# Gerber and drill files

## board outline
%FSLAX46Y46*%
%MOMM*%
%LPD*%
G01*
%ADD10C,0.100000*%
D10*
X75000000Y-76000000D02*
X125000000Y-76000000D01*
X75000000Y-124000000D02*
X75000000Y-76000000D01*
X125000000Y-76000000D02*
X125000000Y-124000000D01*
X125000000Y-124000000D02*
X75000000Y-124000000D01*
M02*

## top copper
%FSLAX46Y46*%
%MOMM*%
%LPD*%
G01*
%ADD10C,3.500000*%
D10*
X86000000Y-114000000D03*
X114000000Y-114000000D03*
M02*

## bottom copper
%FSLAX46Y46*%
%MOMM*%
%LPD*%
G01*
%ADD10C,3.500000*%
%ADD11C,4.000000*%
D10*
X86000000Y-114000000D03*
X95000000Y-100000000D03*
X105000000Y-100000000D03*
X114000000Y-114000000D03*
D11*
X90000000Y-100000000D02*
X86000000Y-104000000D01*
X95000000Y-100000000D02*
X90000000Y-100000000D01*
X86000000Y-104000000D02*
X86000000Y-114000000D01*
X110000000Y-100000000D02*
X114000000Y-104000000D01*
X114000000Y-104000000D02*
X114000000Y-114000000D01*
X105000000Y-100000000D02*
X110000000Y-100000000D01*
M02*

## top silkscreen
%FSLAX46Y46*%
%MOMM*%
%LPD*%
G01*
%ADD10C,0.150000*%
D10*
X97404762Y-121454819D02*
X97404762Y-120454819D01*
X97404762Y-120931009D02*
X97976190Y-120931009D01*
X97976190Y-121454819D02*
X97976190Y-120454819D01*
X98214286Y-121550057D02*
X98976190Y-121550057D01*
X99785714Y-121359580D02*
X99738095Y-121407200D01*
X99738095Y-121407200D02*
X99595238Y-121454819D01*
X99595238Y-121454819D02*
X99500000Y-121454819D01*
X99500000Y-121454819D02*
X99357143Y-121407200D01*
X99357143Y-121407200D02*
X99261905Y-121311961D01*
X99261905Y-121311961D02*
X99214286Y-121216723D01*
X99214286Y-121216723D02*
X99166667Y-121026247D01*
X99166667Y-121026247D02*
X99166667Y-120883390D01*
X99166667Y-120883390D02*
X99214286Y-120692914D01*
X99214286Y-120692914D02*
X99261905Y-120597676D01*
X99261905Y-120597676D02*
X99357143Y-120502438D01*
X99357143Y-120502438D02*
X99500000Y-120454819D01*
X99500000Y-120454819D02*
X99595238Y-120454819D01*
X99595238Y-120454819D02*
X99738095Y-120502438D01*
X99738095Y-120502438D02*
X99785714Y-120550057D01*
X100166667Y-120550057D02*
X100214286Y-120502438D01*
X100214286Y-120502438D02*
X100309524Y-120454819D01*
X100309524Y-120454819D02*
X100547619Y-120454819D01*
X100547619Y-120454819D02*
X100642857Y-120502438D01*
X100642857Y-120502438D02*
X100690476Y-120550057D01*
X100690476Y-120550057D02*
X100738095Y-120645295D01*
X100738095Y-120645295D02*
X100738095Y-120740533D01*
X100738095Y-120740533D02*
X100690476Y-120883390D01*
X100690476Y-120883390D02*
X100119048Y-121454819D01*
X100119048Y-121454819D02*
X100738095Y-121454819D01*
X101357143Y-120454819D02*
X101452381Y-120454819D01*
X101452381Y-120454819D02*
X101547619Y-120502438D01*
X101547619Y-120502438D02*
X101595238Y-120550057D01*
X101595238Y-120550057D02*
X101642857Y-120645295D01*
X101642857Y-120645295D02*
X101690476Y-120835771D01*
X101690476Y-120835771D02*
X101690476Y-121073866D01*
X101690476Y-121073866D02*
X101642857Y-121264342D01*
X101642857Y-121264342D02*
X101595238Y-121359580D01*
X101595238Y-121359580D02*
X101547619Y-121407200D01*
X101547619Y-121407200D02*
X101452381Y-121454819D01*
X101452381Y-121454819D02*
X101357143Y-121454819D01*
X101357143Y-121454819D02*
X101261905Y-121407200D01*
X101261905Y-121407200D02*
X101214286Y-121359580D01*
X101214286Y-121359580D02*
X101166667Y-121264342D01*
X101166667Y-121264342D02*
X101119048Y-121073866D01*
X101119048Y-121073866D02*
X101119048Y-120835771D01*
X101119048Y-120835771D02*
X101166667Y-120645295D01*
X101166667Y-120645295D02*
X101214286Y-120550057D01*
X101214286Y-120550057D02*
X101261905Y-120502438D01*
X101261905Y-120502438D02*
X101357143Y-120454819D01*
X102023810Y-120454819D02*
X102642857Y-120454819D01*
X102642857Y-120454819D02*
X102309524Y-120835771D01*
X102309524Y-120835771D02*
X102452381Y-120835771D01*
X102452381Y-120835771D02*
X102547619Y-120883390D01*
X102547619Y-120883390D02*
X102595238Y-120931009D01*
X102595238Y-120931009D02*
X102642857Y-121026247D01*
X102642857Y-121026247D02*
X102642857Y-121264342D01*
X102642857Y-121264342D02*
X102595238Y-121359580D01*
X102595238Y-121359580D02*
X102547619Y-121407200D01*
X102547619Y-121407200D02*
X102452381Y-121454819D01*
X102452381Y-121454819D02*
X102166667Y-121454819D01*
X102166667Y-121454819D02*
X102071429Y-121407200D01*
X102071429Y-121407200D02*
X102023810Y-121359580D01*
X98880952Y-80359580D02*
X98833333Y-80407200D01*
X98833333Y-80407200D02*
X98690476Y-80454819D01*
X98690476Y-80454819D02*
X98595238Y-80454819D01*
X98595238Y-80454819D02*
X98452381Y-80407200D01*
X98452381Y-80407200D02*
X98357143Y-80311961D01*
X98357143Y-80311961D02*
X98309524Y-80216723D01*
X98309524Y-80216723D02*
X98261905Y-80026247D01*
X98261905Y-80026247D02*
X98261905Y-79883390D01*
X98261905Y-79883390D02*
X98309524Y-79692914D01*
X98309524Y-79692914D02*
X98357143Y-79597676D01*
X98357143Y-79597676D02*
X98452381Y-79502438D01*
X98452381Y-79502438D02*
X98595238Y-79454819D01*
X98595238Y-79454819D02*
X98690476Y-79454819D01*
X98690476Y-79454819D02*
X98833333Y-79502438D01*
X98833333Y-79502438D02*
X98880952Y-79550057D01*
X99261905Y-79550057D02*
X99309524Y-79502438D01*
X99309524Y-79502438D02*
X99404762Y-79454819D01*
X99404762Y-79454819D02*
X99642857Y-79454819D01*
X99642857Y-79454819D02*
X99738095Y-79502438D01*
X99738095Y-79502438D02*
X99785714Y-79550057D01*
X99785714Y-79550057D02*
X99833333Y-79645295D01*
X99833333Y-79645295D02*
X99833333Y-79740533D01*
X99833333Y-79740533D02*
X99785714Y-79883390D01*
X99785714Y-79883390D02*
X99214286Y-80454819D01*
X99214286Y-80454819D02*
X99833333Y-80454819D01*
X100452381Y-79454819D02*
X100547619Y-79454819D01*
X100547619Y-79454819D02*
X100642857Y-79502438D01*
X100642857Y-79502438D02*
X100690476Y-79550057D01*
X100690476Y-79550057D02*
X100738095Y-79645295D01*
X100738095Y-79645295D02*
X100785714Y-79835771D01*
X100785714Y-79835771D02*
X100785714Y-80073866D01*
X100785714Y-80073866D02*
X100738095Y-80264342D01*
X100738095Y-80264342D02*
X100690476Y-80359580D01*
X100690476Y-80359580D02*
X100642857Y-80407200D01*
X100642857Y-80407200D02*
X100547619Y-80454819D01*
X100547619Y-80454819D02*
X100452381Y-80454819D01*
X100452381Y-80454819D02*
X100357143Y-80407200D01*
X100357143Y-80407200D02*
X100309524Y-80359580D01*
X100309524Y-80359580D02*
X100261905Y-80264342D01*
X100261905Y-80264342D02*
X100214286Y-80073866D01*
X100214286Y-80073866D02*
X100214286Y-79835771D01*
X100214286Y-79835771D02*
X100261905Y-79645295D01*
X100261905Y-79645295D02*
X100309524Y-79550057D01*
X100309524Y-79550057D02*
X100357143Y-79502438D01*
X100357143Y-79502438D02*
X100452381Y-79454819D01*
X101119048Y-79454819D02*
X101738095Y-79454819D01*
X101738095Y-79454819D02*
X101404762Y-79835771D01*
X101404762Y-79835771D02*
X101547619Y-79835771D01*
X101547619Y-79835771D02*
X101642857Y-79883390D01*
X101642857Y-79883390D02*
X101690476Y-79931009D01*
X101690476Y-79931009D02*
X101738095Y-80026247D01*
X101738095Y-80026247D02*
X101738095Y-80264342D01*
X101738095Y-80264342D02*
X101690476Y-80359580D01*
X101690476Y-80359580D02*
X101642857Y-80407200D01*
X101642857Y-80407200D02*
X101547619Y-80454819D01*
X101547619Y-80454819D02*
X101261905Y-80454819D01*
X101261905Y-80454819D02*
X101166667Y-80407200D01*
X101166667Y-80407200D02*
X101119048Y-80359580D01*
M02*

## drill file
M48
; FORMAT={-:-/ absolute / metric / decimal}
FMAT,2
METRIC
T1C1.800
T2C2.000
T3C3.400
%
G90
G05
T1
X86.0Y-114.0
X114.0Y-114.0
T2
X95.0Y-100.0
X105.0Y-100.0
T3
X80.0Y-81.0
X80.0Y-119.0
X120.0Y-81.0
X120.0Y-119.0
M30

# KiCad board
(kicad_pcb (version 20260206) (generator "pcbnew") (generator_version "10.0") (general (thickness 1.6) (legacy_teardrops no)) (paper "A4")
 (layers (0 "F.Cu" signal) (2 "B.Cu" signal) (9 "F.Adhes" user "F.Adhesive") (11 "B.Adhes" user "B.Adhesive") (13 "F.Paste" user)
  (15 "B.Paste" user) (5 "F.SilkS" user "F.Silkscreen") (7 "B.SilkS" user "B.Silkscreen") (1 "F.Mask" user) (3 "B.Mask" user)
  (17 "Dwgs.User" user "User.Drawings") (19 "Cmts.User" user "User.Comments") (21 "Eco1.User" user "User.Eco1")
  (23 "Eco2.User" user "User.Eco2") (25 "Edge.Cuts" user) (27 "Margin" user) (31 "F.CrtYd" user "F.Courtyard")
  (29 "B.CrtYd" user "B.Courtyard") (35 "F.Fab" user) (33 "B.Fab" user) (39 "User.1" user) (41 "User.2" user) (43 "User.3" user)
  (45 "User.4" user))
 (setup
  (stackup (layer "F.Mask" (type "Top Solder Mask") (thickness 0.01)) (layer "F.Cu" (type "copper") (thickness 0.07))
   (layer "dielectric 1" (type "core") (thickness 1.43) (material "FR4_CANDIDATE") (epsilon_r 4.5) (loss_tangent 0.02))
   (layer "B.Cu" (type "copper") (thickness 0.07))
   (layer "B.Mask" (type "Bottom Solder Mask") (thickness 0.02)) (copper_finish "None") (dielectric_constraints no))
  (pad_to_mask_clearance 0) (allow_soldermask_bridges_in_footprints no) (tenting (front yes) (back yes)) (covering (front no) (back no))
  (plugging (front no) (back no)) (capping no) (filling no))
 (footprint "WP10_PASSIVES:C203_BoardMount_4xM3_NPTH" (layer "F.Cu") (at 100 100)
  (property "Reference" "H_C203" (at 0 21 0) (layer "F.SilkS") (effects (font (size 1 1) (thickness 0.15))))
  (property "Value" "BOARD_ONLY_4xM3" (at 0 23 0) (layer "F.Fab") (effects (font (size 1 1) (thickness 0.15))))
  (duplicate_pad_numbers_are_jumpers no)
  (pad "" np_thru_hole circle (at -20 -19) (size 3.4 3.4) (drill 3.4) (layers "*.Cu" "*.Mask"))
  (pad "" np_thru_hole circle (at -20 19) (size 3.4 3.4) (drill 3.4) (layers "*.Cu" "*.Mask"))
  (pad "" np_thru_hole circle (at 20 -19) (size 3.4 3.4) (drill 3.4) (layers "*.Cu" "*.Mask"))
  (pad "" np_thru_hole circle (at 20 19) (size 3.4 3.4) (drill 3.4) (layers "*.Cu" "*.Mask")))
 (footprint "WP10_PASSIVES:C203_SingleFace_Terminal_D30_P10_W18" (layer "F.Cu") (at 100 100)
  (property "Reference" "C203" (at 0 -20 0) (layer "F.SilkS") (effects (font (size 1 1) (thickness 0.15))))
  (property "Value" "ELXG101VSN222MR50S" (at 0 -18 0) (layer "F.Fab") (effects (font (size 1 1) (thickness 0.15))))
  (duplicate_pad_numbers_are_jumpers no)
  (pad "1" thru_hole circle (at -14 14) (size 3.5 3.5) (drill 1.8) (layers "*.Cu" "*.Mask") (remove_unused_layers no)
   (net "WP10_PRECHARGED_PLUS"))
  (pad "1" thru_hole circle (at -5 0) (size 3.5 3.5) (drill 2) (layers "*.Cu" "*.Mask") (remove_unused_layers yes) (keep_end_layers no)
   (zone_layer_connections) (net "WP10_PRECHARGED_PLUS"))
  (pad "2" thru_hole circle (at 5 0) (size 3.5 3.5) (drill 2) (layers "*.Cu" "*.Mask") (remove_unused_layers yes) (keep_end_layers no)
   (zone_layer_connections) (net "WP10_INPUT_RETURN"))
  (pad "2" thru_hole circle (at 14 14) (size 3.5 3.5) (drill 1.8) (layers "*.Cu" "*.Mask") (remove_unused_layers no)
   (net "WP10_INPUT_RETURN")))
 (gr_line (start 75 76) (end 125 76) (stroke (width 0.1) (type default)) (layer "Edge.Cuts"))
 (gr_line (start 75 124) (end 75 76) (stroke (width 0.1) (type default)) (layer "Edge.Cuts"))
 (gr_line (start 125 76) (end 125 124) (stroke (width 0.1) (type default)) (layer "Edge.Cuts"))
 (gr_line (start 125 124) (end 75 124) (stroke (width 0.1) (type default)) (layer "Edge.Cuts"))
 (segment (start 90 100) (end 86 104) (width 4) (layer "B.Cu") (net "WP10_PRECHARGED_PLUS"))
 (segment (start 95 100) (end 90 100) (width 4) (layer "B.Cu") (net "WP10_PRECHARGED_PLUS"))
 (segment (start 86 104) (end 86 114) (width 4) (layer "B.Cu") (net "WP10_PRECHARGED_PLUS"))
 (segment (start 110 100) (end 114 104) (width 4) (layer "B.Cu") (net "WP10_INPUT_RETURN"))
 (segment (start 114 104) (end 114 114) (width 4) (layer "B.Cu") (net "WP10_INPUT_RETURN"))
 (segment (start 105 100) (end 110 100) (width 4) (layer "B.Cu") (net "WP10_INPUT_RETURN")))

